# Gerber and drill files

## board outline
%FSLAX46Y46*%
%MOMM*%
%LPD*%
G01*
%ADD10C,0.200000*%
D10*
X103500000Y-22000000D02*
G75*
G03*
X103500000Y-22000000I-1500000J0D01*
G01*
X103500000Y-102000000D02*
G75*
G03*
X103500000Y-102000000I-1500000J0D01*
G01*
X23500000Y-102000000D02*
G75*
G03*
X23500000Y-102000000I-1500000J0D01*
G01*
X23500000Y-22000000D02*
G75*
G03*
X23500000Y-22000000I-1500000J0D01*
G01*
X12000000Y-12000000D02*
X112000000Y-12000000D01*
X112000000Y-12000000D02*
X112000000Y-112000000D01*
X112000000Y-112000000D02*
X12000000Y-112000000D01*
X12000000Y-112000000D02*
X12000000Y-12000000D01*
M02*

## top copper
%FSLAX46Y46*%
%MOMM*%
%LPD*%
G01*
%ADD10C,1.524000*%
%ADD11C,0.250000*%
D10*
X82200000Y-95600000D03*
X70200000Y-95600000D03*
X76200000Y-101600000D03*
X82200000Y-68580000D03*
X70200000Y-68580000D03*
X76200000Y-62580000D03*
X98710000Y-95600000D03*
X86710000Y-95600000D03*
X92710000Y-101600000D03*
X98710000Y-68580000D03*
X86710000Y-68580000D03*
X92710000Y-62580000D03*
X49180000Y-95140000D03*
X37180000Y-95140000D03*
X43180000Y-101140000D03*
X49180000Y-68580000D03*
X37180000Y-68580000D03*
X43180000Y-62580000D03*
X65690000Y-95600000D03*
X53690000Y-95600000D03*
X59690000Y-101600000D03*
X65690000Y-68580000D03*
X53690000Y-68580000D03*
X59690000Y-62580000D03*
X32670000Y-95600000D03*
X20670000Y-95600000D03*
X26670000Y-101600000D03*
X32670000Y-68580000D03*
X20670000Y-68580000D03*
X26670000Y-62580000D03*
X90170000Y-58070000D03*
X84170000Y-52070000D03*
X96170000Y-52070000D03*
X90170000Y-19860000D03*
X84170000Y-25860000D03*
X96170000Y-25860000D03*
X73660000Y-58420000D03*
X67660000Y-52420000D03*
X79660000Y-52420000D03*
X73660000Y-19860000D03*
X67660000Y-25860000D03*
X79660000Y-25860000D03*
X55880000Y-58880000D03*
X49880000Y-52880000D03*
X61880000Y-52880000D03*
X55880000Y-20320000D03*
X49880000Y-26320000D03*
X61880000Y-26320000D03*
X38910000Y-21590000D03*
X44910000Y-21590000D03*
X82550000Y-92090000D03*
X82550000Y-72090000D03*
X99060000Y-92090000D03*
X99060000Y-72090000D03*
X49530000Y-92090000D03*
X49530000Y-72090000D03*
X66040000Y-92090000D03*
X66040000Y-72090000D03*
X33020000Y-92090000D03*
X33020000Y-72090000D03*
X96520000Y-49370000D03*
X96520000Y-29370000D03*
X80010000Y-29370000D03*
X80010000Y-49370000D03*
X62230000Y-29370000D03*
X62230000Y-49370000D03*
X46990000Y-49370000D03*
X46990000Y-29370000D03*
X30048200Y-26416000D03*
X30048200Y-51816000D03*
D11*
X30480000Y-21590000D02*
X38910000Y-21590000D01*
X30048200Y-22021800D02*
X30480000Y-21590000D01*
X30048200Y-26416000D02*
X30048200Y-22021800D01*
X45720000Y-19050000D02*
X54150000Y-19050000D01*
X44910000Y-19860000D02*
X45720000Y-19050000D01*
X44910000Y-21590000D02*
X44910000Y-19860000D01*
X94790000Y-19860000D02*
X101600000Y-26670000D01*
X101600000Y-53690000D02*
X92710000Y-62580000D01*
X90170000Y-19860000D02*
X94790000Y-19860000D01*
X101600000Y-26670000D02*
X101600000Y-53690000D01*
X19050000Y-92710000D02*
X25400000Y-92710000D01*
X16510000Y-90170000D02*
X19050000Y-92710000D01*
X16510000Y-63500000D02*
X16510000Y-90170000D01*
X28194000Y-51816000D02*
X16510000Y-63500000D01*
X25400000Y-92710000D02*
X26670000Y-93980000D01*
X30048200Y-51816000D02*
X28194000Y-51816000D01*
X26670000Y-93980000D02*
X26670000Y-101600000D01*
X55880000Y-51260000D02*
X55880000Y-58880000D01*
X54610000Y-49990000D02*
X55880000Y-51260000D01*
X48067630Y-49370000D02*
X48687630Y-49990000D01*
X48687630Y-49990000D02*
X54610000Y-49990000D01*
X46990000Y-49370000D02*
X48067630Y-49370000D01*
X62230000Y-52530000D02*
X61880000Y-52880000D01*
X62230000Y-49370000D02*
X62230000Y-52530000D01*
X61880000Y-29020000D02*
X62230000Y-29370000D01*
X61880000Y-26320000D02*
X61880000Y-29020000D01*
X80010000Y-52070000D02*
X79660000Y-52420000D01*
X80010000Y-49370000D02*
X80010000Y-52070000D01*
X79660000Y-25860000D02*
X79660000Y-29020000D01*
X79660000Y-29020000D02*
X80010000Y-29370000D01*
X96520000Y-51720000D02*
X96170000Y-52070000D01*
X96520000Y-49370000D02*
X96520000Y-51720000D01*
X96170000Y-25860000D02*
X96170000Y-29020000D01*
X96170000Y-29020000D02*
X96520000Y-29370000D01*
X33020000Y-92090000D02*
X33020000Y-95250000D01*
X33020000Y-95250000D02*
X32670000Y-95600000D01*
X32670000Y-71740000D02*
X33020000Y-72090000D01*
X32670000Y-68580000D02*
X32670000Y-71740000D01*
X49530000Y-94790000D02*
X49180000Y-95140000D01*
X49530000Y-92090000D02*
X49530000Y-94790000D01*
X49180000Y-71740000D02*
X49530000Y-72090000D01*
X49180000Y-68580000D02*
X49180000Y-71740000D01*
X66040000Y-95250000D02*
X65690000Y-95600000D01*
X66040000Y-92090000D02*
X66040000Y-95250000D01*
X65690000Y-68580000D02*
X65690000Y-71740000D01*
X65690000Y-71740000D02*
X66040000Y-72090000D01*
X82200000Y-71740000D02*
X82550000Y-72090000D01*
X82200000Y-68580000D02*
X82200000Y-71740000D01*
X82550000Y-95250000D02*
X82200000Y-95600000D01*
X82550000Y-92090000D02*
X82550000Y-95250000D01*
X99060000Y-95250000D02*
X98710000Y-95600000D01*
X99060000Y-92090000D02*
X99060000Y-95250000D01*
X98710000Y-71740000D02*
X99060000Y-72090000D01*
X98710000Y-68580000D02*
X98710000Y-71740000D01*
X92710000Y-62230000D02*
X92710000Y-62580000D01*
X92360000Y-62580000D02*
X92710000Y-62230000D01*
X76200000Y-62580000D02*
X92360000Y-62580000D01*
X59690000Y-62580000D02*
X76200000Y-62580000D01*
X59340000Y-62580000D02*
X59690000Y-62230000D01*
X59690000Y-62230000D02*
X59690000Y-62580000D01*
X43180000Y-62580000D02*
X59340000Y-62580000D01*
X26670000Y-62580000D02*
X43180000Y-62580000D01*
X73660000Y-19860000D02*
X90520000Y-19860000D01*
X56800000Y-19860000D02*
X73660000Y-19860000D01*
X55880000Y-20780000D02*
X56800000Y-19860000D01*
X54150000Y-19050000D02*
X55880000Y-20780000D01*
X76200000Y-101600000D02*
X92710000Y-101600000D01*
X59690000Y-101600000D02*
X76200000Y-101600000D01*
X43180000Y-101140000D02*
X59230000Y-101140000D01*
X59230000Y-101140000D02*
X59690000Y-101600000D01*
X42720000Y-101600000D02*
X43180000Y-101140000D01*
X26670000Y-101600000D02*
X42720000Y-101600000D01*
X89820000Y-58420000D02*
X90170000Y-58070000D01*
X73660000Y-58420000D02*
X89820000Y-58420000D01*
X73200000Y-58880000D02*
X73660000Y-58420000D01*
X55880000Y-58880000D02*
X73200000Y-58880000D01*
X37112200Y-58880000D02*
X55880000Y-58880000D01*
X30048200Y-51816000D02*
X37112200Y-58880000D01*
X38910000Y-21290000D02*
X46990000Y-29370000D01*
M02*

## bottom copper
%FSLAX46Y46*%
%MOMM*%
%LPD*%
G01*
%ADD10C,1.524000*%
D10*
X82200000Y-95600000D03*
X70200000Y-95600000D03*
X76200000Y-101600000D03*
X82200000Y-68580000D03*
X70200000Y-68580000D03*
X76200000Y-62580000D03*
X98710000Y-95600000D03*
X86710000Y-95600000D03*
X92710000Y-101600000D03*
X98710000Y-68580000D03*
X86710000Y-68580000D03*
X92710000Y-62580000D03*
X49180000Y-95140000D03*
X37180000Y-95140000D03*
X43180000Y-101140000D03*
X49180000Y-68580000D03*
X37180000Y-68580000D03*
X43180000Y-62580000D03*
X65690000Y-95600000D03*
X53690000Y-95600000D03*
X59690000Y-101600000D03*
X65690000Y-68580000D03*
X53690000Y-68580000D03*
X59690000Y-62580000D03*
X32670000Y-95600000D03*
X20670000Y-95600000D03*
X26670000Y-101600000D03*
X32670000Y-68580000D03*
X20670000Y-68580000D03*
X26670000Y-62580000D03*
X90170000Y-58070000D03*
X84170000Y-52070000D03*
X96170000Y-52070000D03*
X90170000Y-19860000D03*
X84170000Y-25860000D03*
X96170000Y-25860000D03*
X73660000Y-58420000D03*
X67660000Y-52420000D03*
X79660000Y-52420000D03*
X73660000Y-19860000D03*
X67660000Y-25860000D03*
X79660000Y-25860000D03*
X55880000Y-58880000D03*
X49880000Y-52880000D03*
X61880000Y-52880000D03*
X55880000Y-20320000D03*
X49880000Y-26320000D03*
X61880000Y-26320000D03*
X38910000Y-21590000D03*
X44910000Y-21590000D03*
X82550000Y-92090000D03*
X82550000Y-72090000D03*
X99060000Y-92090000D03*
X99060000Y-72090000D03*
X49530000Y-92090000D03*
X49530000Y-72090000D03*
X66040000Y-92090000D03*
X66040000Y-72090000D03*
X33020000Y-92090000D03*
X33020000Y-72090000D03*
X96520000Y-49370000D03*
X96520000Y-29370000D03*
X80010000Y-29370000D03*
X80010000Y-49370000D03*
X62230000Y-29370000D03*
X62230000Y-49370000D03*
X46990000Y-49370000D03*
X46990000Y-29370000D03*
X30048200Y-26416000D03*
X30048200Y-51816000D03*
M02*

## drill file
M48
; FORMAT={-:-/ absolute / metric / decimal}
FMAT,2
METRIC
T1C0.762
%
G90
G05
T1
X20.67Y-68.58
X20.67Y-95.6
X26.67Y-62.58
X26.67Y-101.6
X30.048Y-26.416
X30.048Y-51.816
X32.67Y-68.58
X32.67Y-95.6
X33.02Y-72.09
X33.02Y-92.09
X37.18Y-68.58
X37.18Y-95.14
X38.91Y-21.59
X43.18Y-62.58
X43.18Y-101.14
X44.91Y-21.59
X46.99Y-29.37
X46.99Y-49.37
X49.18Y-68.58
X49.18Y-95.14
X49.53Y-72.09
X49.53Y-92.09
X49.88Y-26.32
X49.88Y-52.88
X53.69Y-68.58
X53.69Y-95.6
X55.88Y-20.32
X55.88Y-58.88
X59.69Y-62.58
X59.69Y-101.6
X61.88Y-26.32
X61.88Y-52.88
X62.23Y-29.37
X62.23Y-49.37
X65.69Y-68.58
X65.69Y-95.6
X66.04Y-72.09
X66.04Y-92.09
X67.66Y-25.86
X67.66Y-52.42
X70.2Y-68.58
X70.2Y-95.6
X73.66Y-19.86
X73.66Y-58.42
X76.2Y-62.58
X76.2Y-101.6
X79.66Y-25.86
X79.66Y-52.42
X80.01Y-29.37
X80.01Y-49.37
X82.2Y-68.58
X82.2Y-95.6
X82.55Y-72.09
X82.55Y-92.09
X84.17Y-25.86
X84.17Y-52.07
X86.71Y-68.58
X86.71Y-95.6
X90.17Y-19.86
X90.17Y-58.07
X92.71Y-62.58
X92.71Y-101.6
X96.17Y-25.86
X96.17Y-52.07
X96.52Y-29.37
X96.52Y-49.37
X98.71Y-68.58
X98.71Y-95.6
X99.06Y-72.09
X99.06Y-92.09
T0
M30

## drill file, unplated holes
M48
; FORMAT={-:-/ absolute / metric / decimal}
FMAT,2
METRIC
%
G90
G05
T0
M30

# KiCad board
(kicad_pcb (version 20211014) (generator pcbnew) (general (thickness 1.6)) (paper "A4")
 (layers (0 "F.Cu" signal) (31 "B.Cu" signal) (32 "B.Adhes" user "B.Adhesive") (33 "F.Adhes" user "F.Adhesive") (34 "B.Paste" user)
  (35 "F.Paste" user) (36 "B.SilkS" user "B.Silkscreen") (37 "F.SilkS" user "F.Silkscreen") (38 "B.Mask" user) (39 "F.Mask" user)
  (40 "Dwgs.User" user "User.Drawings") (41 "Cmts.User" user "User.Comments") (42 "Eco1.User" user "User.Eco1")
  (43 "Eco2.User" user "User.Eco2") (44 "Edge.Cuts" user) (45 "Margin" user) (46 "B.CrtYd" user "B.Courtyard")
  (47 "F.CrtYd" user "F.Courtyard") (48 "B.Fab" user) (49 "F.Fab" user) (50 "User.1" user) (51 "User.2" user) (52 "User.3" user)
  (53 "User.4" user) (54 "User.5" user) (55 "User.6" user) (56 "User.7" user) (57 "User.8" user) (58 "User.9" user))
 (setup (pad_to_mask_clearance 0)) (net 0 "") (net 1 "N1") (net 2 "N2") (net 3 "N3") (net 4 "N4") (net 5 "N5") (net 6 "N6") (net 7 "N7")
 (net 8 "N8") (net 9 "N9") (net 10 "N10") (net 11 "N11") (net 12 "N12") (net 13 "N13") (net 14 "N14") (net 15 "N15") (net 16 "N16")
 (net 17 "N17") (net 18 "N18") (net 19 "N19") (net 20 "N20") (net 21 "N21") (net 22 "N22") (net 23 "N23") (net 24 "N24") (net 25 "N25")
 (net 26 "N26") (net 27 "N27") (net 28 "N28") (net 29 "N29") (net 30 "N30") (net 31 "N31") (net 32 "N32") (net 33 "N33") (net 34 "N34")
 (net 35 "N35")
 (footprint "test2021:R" (layer "F.Cu") (at 99.06 82.09 -90)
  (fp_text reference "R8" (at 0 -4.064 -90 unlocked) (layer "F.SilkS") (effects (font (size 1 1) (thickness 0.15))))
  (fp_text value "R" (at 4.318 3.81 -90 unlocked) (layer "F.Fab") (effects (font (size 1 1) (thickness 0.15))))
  (pad "1" thru_hole circle (at -10 0 270) (size 1.524 1.524) (drill 0.762) (layers *.Cu *.Mask) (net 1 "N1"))
  (pad "2" thru_hole circle (at 10 0 270) (size 1.524 1.524) (drill 0.762) (layers *.Cu *.Mask) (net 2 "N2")))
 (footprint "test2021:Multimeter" (layer "F.Cu") (at 41.91 21.59 90)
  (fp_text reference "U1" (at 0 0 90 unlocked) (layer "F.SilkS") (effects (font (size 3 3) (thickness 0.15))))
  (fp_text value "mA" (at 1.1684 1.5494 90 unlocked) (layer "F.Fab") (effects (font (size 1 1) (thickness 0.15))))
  (pad "1" thru_hole circle (at 0 -3 90) (size 1.524 1.524) (drill 0.762) (layers *.Cu *.Mask) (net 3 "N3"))
  (pad "2" thru_hole circle (at 0 3 90) (size 1.524 1.524) (drill 0.762) (layers *.Cu *.Mask) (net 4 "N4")))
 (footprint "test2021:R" (layer "F.Cu") (at 66.04 82.09 -90)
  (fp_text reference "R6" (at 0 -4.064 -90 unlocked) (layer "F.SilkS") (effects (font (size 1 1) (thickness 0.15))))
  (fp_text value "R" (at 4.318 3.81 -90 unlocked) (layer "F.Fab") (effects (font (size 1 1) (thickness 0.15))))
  (pad "1" thru_hole circle (at -10 0 270) (size 1.524 1.524) (drill 0.762) (layers *.Cu *.Mask) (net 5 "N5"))
  (pad "2" thru_hole circle (at 10 0 270) (size 1.524 1.524) (drill 0.762) (layers *.Cu *.Mask) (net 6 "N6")))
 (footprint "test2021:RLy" (layer "F.Cu") (at 43.18 68.58)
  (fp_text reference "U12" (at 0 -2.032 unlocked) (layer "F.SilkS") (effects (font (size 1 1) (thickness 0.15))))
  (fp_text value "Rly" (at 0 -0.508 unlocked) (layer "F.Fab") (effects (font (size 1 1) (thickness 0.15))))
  (pad "1" thru_hole circle (at 0 -6) (size 1.524 1.524) (drill 0.762) (layers *.Cu *.Mask) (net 4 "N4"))
  (pad "2" thru_hole circle (at -6 0) (size 1.524 1.524) (drill 0.762) (layers *.Cu *.Mask) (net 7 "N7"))
  (pad "3" thru_hole circle (at 6 0) (size 1.524 1.524) (drill 0.762) (layers *.Cu *.Mask) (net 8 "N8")))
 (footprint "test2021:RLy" (layer "F.Cu") (at 90.17 25.86)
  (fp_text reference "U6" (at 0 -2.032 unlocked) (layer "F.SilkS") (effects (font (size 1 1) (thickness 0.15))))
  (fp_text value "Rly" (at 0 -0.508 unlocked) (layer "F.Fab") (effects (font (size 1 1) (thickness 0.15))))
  (pad "1" thru_hole circle (at 0 -6) (size 1.524 1.524) (drill 0.762) (layers *.Cu *.Mask) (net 4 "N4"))
  (pad "2" thru_hole circle (at -6 0) (size 1.524 1.524) (drill 0.762) (layers *.Cu *.Mask) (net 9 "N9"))
  (pad "3" thru_hole circle (at 6 0) (size 1.524 1.524) (drill 0.762) (layers *.Cu *.Mask) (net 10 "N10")))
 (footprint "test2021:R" (layer "F.Cu") (at 62.23 39.37 -90)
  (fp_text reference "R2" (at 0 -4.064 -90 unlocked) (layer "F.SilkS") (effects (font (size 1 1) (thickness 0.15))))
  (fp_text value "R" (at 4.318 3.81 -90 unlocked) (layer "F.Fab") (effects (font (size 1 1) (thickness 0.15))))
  (pad "1" thru_hole circle (at -10 0 270) (size 1.524 1.524) (drill 0.762) (layers *.Cu *.Mask) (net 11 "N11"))
  (pad "2" thru_hole circle (at 10 0 270) (size 1.524 1.524) (drill 0.762) (layers *.Cu *.Mask) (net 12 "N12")))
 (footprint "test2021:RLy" (layer "F.Cu") (at 76.2 68.58)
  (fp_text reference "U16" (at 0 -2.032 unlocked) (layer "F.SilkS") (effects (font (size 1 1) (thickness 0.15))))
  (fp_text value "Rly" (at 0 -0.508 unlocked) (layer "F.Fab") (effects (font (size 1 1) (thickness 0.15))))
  (pad "1" thru_hole circle (at 0 -6) (size 1.524 1.524) (drill 0.762) (layers *.Cu *.Mask) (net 4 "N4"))
  (pad "2" thru_hole circle (at -6 0) (size 1.524 1.524) (drill 0.762) (layers *.Cu *.Mask) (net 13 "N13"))
  (pad "3" thru_hole circle (at 6 0) (size 1.524 1.524) (drill 0.762) (layers *.Cu *.Mask) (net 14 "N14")))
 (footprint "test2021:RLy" (layer "F.Cu") (at 73.66 25.86)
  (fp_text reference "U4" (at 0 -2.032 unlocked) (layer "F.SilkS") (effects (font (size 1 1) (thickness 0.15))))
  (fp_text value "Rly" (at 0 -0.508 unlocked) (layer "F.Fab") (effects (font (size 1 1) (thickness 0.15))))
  (pad "1" thru_hole circle (at 0 -6) (size 1.524 1.524) (drill 0.762) (layers *.Cu *.Mask) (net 4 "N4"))
  (pad "2" thru_hole circle (at -6 0) (size 1.524 1.524) (drill 0.762) (layers *.Cu *.Mask) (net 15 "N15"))
  (pad "3" thru_hole circle (at 6 0) (size 1.524 1.524) (drill 0.762) (layers *.Cu *.Mask) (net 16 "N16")))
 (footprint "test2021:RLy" (layer "F.Cu") (at 59.69 68.58)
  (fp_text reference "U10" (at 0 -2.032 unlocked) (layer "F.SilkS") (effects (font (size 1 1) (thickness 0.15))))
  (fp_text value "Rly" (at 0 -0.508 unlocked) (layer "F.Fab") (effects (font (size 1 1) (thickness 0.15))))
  (pad "1" thru_hole circle (at 0 -6) (size 1.524 1.524) (drill 0.762) (layers *.Cu *.Mask) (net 4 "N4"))
  (pad "2" thru_hole circle (at -6 0) (size 1.524 1.524) (drill 0.762) (layers *.Cu *.Mask) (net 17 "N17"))
  (pad "3" thru_hole circle (at 6 0) (size 1.524 1.524) (drill 0.762) (layers *.Cu *.Mask) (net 5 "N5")))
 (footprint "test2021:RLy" (layer "F.Cu") (at 26.67 68.58)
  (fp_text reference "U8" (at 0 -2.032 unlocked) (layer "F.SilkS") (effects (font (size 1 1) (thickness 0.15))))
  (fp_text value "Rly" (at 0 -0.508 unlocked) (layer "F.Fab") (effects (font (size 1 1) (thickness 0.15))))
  (pad "1" thru_hole circle (at 0 -6) (size 1.524 1.524) (drill 0.762) (layers *.Cu *.Mask) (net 4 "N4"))
  (pad "2" thru_hole circle (at -6 0) (size 1.524 1.524) (drill 0.762) (layers *.Cu *.Mask) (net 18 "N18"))
  (pad "3" thru_hole circle (at 6 0) (size 1.524 1.524) (drill 0.762) (layers *.Cu *.Mask) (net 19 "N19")))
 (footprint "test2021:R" (layer "F.Cu") (at 82.55 82.09 -90)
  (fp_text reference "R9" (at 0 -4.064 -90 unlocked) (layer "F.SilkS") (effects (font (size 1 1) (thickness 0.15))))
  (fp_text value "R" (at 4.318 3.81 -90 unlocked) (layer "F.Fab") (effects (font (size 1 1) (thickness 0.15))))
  (pad "1" thru_hole circle (at -10 0 270) (size 1.524 1.524) (drill 0.762) (layers *.Cu *.Mask) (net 14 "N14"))
  (pad "2" thru_hole circle (at 10 0 270) (size 1.524 1.524) (drill 0.762) (layers *.Cu *.Mask) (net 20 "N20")))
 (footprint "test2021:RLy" (layer "F.Cu") (at 55.88 26.32)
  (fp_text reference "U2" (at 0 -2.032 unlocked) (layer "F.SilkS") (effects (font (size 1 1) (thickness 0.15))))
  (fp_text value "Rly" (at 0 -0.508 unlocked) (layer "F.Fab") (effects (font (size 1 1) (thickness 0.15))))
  (pad "1" thru_hole circle (at 0 -6) (size 1.524 1.524) (drill 0.762) (layers *.Cu *.Mask) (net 4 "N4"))
  (pad "2" thru_hole circle (at -6 0) (size 1.524 1.524) (drill 0.762) (layers *.Cu *.Mask) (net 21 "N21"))
  (pad "3" thru_hole circle (at 6 0) (size 1.524 1.524) (drill 0.762) (layers *.Cu *.Mask) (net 11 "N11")))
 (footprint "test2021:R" (layer "F.Cu") (at 46.99 39.37 -90)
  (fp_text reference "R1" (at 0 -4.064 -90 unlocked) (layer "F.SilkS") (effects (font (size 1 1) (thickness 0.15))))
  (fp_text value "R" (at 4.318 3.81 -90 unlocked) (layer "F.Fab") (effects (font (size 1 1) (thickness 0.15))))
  (pad "1" thru_hole circle (at -10 0 270) (size 1.524 1.524) (drill 0.762) (layers *.Cu *.Mask) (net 3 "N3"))
  (pad "2" thru_hole circle (at 10 0 270) (size 1.524 1.524) (drill 0.762) (layers *.Cu *.Mask) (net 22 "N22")))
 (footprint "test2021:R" (layer "F.Cu") (at 49.53 82.09 -90)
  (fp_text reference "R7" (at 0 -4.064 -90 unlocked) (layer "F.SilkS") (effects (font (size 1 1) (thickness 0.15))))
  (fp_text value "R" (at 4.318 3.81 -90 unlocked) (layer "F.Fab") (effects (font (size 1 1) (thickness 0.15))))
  (pad "1" thru_hole circle (at -10 0 270) (size 1.524 1.524) (drill 0.762) (layers *.Cu *.Mask) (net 8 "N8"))
  (pad "2" thru_hole circle (at 10 0 270) (size 1.524 1.524) (drill 0.762) (layers *.Cu *.Mask) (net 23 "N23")))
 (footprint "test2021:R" (layer "F.Cu") (at 33.02 82.09 -90)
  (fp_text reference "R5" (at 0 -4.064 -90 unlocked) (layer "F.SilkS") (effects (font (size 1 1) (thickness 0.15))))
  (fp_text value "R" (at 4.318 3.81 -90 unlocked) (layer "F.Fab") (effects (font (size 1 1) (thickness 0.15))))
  (pad "1" thru_hole circle (at -10 0 270) (size 1.524 1.524) (drill 0.762) (layers *.Cu *.Mask) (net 19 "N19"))
  (pad "2" thru_hole circle (at 10 0 270) (size 1.524 1.524) (drill 0.762) (layers *.Cu *.Mask) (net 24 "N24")))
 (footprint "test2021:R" (layer "F.Cu") (at 96.52 39.37 -90)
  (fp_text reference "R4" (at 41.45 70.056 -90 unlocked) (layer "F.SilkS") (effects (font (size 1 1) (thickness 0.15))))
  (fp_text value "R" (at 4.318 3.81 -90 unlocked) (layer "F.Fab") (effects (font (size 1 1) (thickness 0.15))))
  (pad "1" thru_hole circle (at -10 0 270) (size 1.524 1.524) (drill 0.762) (layers *.Cu *.Mask) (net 10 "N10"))
  (pad "2" thru_hole circle (at 10 0 270) (size 1.524 1.524) (drill 0.762) (layers *.Cu *.Mask) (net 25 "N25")))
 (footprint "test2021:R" (layer "F.Cu") (at 80.01 39.37 -90)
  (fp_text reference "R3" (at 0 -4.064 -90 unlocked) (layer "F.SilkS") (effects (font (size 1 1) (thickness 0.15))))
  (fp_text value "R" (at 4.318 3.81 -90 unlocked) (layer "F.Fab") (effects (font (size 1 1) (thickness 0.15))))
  (pad "1" thru_hole circle (at -10 0 270) (size 1.524 1.524) (drill 0.762) (layers *.Cu *.Mask) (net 16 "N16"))
  (pad "2" thru_hole circle (at 10 0 270) (size 1.524 1.524) (drill 0.762) (layers *.Cu *.Mask) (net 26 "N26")))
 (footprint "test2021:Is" (layer "F.Cu") (at 30.0482 39.116 -90)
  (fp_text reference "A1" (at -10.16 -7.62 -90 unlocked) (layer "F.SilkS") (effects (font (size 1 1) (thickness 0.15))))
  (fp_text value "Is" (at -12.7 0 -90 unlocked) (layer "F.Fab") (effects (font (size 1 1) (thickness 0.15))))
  (pad "1" thru_hole circle (at -12.7 0 270) (size 1.524 1.524) (drill 0.762) (layers *.Cu *.Mask) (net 3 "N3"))
  (pad "2" thru_hole circle (at 12.7 0 270) (size 1.524 1.524) (drill 0.762) (layers *.Cu *.Mask) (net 22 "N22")))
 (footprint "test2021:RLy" (layer "F.Cu") (at 92.71 68.58)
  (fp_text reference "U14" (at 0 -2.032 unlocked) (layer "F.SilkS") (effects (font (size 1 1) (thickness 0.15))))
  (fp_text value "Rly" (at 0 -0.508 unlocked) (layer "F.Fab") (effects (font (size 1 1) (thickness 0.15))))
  (pad "1" thru_hole circle (at 0 -6) (size 1.524 1.524) (drill 0.762) (layers *.Cu *.Mask) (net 4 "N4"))
  (pad "2" thru_hole circle (at -6 0) (size 1.524 1.524) (drill 0.762) (layers *.Cu *.Mask) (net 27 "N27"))
  (pad "3" thru_hole circle (at 6 0) (size 1.524 1.524) (drill 0.762) (layers *.Cu *.Mask) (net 1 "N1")))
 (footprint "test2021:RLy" (layer "B.Cu") (at 90.17 52.07)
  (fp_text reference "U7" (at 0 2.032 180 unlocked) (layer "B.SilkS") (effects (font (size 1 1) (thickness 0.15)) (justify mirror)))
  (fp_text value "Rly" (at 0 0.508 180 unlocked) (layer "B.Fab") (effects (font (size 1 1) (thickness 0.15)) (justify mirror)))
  (pad "1" thru_hole circle (at 0 6) (size 1.524 1.524) (drill 0.762) (layers *.Cu *.Mask) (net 22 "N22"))
  (pad "2" thru_hole circle (at -6 0) (size 1.524 1.524) (drill 0.762) (layers *.Cu *.Mask) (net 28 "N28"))
  (pad "3" thru_hole circle (at 6 0) (size 1.524 1.524) (drill 0.762) (layers *.Cu *.Mask) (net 25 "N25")))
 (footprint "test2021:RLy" (layer "B.Cu") (at 76.2 95.6)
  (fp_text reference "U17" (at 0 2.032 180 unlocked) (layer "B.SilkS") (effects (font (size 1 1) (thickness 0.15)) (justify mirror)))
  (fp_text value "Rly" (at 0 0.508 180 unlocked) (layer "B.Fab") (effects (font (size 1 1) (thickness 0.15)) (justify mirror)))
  (pad "1" thru_hole circle (at 0 6) (size 1.524 1.524) (drill 0.762) (layers *.Cu *.Mask) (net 22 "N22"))
  (pad "2" thru_hole circle (at -6 0) (size 1.524 1.524) (drill 0.762) (layers *.Cu *.Mask) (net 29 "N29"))
  (pad "3" thru_hole circle (at 6 0) (size 1.524 1.524) (drill 0.762) (layers *.Cu *.Mask) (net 20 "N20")))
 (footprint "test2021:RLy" (layer "B.Cu") (at 92.71 95.6)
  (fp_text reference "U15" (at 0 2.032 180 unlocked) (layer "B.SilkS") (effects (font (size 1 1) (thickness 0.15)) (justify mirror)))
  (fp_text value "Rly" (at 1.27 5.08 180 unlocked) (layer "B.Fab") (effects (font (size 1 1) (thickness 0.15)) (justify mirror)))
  (pad "1" thru_hole circle (at 0 6) (size 1.524 1.524) (drill 0.762) (layers *.Cu *.Mask) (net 22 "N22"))
  (pad "2" thru_hole circle (at -6 0) (size 1.524 1.524) (drill 0.762) (layers *.Cu *.Mask) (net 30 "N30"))
  (pad "3" thru_hole circle (at 6 0) (size 1.524 1.524) (drill 0.762) (layers *.Cu *.Mask) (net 2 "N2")))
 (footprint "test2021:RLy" (layer "B.Cu") (at 59.69 95.6)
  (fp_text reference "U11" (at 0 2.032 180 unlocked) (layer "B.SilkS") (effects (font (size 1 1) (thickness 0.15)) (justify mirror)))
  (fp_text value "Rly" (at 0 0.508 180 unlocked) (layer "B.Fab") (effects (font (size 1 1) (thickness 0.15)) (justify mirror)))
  (pad "1" thru_hole circle (at 0 6) (size 1.524 1.524) (drill 0.762) (layers *.Cu *.Mask) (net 22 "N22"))
  (pad "2" thru_hole circle (at -6 0) (size 1.524 1.524) (drill 0.762) (layers *.Cu *.Mask) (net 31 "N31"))
  (pad "3" thru_hole circle (at 6 0) (size 1.524 1.524) (drill 0.762) (layers *.Cu *.Mask) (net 6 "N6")))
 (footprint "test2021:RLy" (layer "B.Cu") (at 73.66 52.42)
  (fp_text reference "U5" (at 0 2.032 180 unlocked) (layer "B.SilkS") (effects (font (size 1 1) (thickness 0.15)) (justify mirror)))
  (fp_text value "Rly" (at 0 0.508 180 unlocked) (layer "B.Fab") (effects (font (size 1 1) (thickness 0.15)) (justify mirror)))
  (pad "1" thru_hole circle (at 0 6) (size 1.524 1.524) (drill 0.762) (layers *.Cu *.Mask) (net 22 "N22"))
  (pad "2" thru_hole circle (at -6 0) (size 1.524 1.524) (drill 0.762) (layers *.Cu *.Mask) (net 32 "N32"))
  (pad "3" thru_hole circle (at 6 0) (size 1.524 1.524) (drill 0.762) (layers *.Cu *.Mask) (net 26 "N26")))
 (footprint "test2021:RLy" (layer "B.Cu") (at 43.18 95.14)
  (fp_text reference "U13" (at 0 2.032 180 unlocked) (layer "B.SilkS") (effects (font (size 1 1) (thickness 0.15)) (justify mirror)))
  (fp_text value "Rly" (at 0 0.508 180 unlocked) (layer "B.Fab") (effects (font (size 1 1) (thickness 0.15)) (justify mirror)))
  (pad "1" thru_hole circle (at 0 6) (size 1.524 1.524) (drill 0.762) (layers *.Cu *.Mask) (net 22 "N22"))
  (pad "2" thru_hole circle (at -6 0) (size 1.524 1.524) (drill 0.762) (layers *.Cu *.Mask) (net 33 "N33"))
  (pad "3" thru_hole circle (at 6 0) (size 1.524 1.524) (drill 0.762) (layers *.Cu *.Mask) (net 23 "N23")))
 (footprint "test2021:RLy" (layer "B.Cu") (at 26.67 95.6)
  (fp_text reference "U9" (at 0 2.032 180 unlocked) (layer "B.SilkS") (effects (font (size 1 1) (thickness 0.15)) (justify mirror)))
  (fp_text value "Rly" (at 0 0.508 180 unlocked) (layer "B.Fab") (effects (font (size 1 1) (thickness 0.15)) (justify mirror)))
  (pad "1" thru_hole circle (at 0 6) (size 1.524 1.524) (drill 0.762) (layers *.Cu *.Mask) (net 22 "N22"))
  (pad "2" thru_hole circle (at -6 0) (size 1.524 1.524) (drill 0.762) (layers *.Cu *.Mask) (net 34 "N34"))
  (pad "3" thru_hole circle (at 6 0) (size 1.524 1.524) (drill 0.762) (layers *.Cu *.Mask) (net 24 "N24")))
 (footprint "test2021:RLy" (layer "B.Cu") (at 55.88 52.88)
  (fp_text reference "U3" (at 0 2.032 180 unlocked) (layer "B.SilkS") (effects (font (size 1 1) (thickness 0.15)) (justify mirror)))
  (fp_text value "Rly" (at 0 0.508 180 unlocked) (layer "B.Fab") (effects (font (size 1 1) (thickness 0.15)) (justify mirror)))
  (pad "1" thru_hole circle (at 0 6) (size 1.524 1.524) (drill 0.762) (layers *.Cu *.Mask) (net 22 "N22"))
  (pad "2" thru_hole circle (at -6 0) (size 1.524 1.524) (drill 0.762) (layers *.Cu *.Mask) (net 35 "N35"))
  (pad "3" thru_hole circle (at 6 0) (size 1.524 1.524) (drill 0.762) (layers *.Cu *.Mask) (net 12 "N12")))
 (gr_circle (center 22 22) (end 23.5 22) (layer "Edge.Cuts") (width 0.2) (fill none))
 (gr_circle (center 22 102) (end 23.5 102) (layer "Edge.Cuts") (width 0.2) (fill none))
 (gr_rect (start 12 12) (end 112 112) (layer "Edge.Cuts") (width 0.2) (fill none))
 (gr_circle (center 102 102) (end 103.5 102) (layer "Edge.Cuts") (width 0.2) (fill none))
 (gr_circle (center 102 22) (end 103.5 22) (layer "Edge.Cuts") (width 0.2) (fill none))
 (segment (start 46.99 49.37) (end 48.06763 49.37) (width 0.25) (layer "F.Cu") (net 22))
 (segment (start 42.72 101.6) (end 43.18 101.14) (width 0.25) (layer "F.Cu") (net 22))
 (segment (start 89.82 58.42) (end 90.17 58.07) (width 0.25) (layer "F.Cu") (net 22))
 (segment (start 26.67 93.98) (end 26.67 101.6) (width 0.25) (layer "F.Cu") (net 22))
 (segment (start 19.05 92.71) (end 25.4 92.71) (width 0.25) (layer "F.Cu") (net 22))
 (segment (start 55.88 58.88) (end 73.2 58.88) (width 0.25) (layer "F.Cu") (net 22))
 (segment (start 76.2 101.6) (end 92.71 101.6) (width 0.25) (layer "F.Cu") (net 22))
 (segment (start 54.61 49.99) (end 55.88 51.26) (width 0.25) (layer "F.Cu") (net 22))
 (segment (start 28.194 51.816) (end 16.51 63.5) (width 0.25) (layer "F.Cu") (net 22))
 (segment (start 73.66 58.42) (end 89.82 58.42) (width 0.25) (layer "F.Cu") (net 22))
 (segment (start 26.67 101.6) (end 42.72 101.6) (width 0.25) (layer "F.Cu") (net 22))
 (segment (start 55.88 51.26) (end 55.88 58.88) (width 0.25) (layer "F.Cu") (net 22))
 (segment (start 37.1122 58.88) (end 55.88 58.88) (width 0.25) (layer "F.Cu") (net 22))
 (segment (start 30.0482 51.816) (end 28.194 51.816) (width 0.25) (layer "F.Cu") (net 22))
 (segment (start 25.4 92.71) (end 26.67 93.98) (width 0.25) (layer "F.Cu") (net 22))
 (segment (start 48.68763 49.99) (end 54.61 49.99) (width 0.25) (layer "F.Cu") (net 22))
 (segment (start 16.51 90.17) (end 19.05 92.71) (width 0.25) (layer "F.Cu") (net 22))
 (segment (start 43.18 101.14) (end 59.23 101.14) (width 0.25) (layer "F.Cu") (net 22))
 (segment (start 48.06763 49.37) (end 48.68763 49.99) (width 0.25) (layer "F.Cu") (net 22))
 (segment (start 59.23 101.14) (end 59.69 101.6) (width 0.25) (layer "F.Cu") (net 22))
 (segment (start 59.69 101.6) (end 76.2 101.6) (width 0.25) (layer "F.Cu") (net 22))
 (segment (start 30.0482 51.816) (end 37.1122 58.88) (width 0.25) (layer "F.Cu") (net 22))
 (segment (start 73.2 58.88) (end 73.66 58.42) (width 0.25) (layer "F.Cu") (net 22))
 (segment (start 16.51 63.5) (end 16.51 90.17) (width 0.25) (layer "F.Cu") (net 22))
 (segment (start 79.66 25.86) (end 79.66 29.02) (width 0.25) (layer "F.Cu") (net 16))
 (segment (start 79.66 29.02) (end 80.01 29.37) (width 0.25) (layer "F.Cu") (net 16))
 (segment (start 80.01 49.37) (end 80.01 52.07) (width 0.25) (layer "F.Cu") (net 26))
 (segment (start 80.01 52.07) (end 79.66 52.42) (width 0.25) (layer "F.Cu") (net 26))
 (segment (start 66.04 92.09) (end 66.04 95.25) (width 0.25) (layer "F.Cu") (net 6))
 (segment (start 66.04 95.25) (end 65.69 95.6) (width 0.25) (layer "F.Cu") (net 6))
 (segment (start 30.0482 22.0218) (end 30.48 21.59) (width 0.25) (layer "F.Cu") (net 3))
 (segment (start 30.48 21.59) (end 38.91 21.59) (width 0.25) (layer "F.Cu") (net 3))
 (segment (start 38.91 21.29) (end 46.99 29.37) (width 0.25) (layer "F.Cu") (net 3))
 (segment (start 30.0482 26.416) (end 30.0482 22.0218) (width 0.25) (layer "F.Cu") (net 3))
 (segment (start 61.88 29.02) (end 62.23 29.37) (width 0.25) (layer "F.Cu") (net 11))
 (segment (start 61.88 26.32) (end 61.88 29.02) (width 0.25) (layer "F.Cu") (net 11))
 (segment (start 62.23 52.53) (end 61.88 52.88) (width 0.25) (layer "F.Cu") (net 12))
 (segment (start 62.23 49.37) (end 62.23 52.53) (width 0.25) (layer "F.Cu") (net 12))
 (segment (start 96.17 25.86) (end 96.17 29.02) (width 0.25) (layer "F.Cu") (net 10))
 (segment (start 96.17 29.02) (end 96.52 29.37) (width 0.25) (layer "F.Cu") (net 10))
 (segment (start 96.52 51.72) (end 96.17 52.07) (width 0.25) (layer "F.Cu") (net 25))
 (segment (start 96.52 49.37) (end 96.52 51.72) (width 0.25) (layer "F.Cu") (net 25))
 (segment (start 32.67 71.74) (end 33.02 72.09) (width 0.25) (layer "F.Cu") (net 19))
 (segment (start 32.67 68.58) (end 32.67 71.74) (width 0.25) (layer "F.Cu") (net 19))
 (segment (start 33.02 92.09) (end 33.02 95.25) (width 0.25) (layer "F.Cu") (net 24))
 (segment (start 33.02 95.25) (end 32.67 95.6) (width 0.25) (layer "F.Cu") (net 24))
 (segment (start 65.69 68.58) (end 65.69 71.74) (width 0.25) (layer "F.Cu") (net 5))
 (segment (start 65.69 71.74) (end 66.04 72.09) (width 0.25) (layer "F.Cu") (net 5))
 (segment (start 49.18 71.74) (end 49.53 72.09) (width 0.25) (layer "F.Cu") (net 8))
 (segment (start 49.18 68.58) (end 49.18 71.74) (width 0.25) (layer "F.Cu") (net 8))
 (segment (start 49.53 92.09) (end 49.53 94.79) (width 0.25) (layer "F.Cu") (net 23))
 (segment (start 49.53 94.79) (end 49.18 95.14) (width 0.25) (layer "F.Cu") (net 23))
 (segment (start 98.71 71.74) (end 99.06 72.09) (width 0.25) (layer "F.Cu") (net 1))
 (segment (start 98.71 68.58) (end 98.71 71.74) (width 0.25) (layer "F.Cu") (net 1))
 (segment (start 99.06 95.25) (end 98.71 95.6) (width 0.25) (layer "F.Cu") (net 2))
 (segment (start 99.06 92.09) (end 99.06 95.25) (width 0.25) (layer "F.Cu") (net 2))
 (segment (start 82.2 71.74) (end 82.55 72.09) (width 0.25) (layer "F.Cu") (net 14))
 (segment (start 82.2 68.58) (end 82.2 71.74) (width 0.25) (layer "F.Cu") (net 14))
 (segment (start 82.55 92.09) (end 82.55 95.25) (width 0.25) (layer "F.Cu") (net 20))
 (segment (start 82.55 95.25) (end 82.2 95.6) (width 0.25) (layer "F.Cu") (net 20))
 (segment (start 43.18 62.58) (end 59.34 62.58) (width 0.25) (layer "F.Cu") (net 4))
 (segment (start 59.69 62.23) (end 59.69 62.58) (width 0.25) (layer "F.Cu") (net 4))
 (segment (start 54.15 19.05) (end 55.88 20.78) (width 0.25) (layer "F.Cu") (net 4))
 (segment (start 101.6 26.67) (end 101.6 53.69) (width 0.25) (layer "F.Cu") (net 4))
 (segment (start 90.17 19.86) (end 94.79 19.86) (width 0.25) (layer "F.Cu") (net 4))
 (segment (start 26.67 62.58) (end 43.18 62.58) (width 0.25) (layer "F.Cu") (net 4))
 (segment (start 73.66 19.86) (end 90.52 19.86) (width 0.25) (layer "F.Cu") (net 4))
 (segment (start 94.79 19.86) (end 101.6 26.67) (width 0.25) (layer "F.Cu") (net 4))
 (segment (start 92.36 62.58) (end 92.71 62.23) (width 0.25) (layer "F.Cu") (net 4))
 (segment (start 59.34 62.58) (end 59.69 62.23) (width 0.25) (layer "F.Cu") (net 4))
 (segment (start 101.6 53.69) (end 92.71 62.58) (width 0.25) (layer "F.Cu") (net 4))
 (segment (start 45.72 19.05) (end 54.15 19.05) (width 0.25) (layer "F.Cu") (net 4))
 (segment (start 44.91 21.59) (end 44.91 19.86) (width 0.25) (layer "F.Cu") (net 4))
 (segment (start 55.88 20.78) (end 56.8 19.86) (width 0.25) (layer "F.Cu") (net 4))
 (segment (start 92.71 62.23) (end 92.71 62.58) (width 0.25) (layer "F.Cu") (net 4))
 (segment (start 44.91 19.86) (end 45.72 19.05) (width 0.25) (layer "F.Cu") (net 4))
 (segment (start 59.69 62.58) (end 76.2 62.58) (width 0.25) (layer "F.Cu") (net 4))
 (segment (start 56.8 19.86) (end 73.66 19.86) (width 0.25) (layer "F.Cu") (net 4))
 (segment (start 76.2 62.58) (end 92.36 62.58) (width 0.25) (layer "F.Cu") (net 4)))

